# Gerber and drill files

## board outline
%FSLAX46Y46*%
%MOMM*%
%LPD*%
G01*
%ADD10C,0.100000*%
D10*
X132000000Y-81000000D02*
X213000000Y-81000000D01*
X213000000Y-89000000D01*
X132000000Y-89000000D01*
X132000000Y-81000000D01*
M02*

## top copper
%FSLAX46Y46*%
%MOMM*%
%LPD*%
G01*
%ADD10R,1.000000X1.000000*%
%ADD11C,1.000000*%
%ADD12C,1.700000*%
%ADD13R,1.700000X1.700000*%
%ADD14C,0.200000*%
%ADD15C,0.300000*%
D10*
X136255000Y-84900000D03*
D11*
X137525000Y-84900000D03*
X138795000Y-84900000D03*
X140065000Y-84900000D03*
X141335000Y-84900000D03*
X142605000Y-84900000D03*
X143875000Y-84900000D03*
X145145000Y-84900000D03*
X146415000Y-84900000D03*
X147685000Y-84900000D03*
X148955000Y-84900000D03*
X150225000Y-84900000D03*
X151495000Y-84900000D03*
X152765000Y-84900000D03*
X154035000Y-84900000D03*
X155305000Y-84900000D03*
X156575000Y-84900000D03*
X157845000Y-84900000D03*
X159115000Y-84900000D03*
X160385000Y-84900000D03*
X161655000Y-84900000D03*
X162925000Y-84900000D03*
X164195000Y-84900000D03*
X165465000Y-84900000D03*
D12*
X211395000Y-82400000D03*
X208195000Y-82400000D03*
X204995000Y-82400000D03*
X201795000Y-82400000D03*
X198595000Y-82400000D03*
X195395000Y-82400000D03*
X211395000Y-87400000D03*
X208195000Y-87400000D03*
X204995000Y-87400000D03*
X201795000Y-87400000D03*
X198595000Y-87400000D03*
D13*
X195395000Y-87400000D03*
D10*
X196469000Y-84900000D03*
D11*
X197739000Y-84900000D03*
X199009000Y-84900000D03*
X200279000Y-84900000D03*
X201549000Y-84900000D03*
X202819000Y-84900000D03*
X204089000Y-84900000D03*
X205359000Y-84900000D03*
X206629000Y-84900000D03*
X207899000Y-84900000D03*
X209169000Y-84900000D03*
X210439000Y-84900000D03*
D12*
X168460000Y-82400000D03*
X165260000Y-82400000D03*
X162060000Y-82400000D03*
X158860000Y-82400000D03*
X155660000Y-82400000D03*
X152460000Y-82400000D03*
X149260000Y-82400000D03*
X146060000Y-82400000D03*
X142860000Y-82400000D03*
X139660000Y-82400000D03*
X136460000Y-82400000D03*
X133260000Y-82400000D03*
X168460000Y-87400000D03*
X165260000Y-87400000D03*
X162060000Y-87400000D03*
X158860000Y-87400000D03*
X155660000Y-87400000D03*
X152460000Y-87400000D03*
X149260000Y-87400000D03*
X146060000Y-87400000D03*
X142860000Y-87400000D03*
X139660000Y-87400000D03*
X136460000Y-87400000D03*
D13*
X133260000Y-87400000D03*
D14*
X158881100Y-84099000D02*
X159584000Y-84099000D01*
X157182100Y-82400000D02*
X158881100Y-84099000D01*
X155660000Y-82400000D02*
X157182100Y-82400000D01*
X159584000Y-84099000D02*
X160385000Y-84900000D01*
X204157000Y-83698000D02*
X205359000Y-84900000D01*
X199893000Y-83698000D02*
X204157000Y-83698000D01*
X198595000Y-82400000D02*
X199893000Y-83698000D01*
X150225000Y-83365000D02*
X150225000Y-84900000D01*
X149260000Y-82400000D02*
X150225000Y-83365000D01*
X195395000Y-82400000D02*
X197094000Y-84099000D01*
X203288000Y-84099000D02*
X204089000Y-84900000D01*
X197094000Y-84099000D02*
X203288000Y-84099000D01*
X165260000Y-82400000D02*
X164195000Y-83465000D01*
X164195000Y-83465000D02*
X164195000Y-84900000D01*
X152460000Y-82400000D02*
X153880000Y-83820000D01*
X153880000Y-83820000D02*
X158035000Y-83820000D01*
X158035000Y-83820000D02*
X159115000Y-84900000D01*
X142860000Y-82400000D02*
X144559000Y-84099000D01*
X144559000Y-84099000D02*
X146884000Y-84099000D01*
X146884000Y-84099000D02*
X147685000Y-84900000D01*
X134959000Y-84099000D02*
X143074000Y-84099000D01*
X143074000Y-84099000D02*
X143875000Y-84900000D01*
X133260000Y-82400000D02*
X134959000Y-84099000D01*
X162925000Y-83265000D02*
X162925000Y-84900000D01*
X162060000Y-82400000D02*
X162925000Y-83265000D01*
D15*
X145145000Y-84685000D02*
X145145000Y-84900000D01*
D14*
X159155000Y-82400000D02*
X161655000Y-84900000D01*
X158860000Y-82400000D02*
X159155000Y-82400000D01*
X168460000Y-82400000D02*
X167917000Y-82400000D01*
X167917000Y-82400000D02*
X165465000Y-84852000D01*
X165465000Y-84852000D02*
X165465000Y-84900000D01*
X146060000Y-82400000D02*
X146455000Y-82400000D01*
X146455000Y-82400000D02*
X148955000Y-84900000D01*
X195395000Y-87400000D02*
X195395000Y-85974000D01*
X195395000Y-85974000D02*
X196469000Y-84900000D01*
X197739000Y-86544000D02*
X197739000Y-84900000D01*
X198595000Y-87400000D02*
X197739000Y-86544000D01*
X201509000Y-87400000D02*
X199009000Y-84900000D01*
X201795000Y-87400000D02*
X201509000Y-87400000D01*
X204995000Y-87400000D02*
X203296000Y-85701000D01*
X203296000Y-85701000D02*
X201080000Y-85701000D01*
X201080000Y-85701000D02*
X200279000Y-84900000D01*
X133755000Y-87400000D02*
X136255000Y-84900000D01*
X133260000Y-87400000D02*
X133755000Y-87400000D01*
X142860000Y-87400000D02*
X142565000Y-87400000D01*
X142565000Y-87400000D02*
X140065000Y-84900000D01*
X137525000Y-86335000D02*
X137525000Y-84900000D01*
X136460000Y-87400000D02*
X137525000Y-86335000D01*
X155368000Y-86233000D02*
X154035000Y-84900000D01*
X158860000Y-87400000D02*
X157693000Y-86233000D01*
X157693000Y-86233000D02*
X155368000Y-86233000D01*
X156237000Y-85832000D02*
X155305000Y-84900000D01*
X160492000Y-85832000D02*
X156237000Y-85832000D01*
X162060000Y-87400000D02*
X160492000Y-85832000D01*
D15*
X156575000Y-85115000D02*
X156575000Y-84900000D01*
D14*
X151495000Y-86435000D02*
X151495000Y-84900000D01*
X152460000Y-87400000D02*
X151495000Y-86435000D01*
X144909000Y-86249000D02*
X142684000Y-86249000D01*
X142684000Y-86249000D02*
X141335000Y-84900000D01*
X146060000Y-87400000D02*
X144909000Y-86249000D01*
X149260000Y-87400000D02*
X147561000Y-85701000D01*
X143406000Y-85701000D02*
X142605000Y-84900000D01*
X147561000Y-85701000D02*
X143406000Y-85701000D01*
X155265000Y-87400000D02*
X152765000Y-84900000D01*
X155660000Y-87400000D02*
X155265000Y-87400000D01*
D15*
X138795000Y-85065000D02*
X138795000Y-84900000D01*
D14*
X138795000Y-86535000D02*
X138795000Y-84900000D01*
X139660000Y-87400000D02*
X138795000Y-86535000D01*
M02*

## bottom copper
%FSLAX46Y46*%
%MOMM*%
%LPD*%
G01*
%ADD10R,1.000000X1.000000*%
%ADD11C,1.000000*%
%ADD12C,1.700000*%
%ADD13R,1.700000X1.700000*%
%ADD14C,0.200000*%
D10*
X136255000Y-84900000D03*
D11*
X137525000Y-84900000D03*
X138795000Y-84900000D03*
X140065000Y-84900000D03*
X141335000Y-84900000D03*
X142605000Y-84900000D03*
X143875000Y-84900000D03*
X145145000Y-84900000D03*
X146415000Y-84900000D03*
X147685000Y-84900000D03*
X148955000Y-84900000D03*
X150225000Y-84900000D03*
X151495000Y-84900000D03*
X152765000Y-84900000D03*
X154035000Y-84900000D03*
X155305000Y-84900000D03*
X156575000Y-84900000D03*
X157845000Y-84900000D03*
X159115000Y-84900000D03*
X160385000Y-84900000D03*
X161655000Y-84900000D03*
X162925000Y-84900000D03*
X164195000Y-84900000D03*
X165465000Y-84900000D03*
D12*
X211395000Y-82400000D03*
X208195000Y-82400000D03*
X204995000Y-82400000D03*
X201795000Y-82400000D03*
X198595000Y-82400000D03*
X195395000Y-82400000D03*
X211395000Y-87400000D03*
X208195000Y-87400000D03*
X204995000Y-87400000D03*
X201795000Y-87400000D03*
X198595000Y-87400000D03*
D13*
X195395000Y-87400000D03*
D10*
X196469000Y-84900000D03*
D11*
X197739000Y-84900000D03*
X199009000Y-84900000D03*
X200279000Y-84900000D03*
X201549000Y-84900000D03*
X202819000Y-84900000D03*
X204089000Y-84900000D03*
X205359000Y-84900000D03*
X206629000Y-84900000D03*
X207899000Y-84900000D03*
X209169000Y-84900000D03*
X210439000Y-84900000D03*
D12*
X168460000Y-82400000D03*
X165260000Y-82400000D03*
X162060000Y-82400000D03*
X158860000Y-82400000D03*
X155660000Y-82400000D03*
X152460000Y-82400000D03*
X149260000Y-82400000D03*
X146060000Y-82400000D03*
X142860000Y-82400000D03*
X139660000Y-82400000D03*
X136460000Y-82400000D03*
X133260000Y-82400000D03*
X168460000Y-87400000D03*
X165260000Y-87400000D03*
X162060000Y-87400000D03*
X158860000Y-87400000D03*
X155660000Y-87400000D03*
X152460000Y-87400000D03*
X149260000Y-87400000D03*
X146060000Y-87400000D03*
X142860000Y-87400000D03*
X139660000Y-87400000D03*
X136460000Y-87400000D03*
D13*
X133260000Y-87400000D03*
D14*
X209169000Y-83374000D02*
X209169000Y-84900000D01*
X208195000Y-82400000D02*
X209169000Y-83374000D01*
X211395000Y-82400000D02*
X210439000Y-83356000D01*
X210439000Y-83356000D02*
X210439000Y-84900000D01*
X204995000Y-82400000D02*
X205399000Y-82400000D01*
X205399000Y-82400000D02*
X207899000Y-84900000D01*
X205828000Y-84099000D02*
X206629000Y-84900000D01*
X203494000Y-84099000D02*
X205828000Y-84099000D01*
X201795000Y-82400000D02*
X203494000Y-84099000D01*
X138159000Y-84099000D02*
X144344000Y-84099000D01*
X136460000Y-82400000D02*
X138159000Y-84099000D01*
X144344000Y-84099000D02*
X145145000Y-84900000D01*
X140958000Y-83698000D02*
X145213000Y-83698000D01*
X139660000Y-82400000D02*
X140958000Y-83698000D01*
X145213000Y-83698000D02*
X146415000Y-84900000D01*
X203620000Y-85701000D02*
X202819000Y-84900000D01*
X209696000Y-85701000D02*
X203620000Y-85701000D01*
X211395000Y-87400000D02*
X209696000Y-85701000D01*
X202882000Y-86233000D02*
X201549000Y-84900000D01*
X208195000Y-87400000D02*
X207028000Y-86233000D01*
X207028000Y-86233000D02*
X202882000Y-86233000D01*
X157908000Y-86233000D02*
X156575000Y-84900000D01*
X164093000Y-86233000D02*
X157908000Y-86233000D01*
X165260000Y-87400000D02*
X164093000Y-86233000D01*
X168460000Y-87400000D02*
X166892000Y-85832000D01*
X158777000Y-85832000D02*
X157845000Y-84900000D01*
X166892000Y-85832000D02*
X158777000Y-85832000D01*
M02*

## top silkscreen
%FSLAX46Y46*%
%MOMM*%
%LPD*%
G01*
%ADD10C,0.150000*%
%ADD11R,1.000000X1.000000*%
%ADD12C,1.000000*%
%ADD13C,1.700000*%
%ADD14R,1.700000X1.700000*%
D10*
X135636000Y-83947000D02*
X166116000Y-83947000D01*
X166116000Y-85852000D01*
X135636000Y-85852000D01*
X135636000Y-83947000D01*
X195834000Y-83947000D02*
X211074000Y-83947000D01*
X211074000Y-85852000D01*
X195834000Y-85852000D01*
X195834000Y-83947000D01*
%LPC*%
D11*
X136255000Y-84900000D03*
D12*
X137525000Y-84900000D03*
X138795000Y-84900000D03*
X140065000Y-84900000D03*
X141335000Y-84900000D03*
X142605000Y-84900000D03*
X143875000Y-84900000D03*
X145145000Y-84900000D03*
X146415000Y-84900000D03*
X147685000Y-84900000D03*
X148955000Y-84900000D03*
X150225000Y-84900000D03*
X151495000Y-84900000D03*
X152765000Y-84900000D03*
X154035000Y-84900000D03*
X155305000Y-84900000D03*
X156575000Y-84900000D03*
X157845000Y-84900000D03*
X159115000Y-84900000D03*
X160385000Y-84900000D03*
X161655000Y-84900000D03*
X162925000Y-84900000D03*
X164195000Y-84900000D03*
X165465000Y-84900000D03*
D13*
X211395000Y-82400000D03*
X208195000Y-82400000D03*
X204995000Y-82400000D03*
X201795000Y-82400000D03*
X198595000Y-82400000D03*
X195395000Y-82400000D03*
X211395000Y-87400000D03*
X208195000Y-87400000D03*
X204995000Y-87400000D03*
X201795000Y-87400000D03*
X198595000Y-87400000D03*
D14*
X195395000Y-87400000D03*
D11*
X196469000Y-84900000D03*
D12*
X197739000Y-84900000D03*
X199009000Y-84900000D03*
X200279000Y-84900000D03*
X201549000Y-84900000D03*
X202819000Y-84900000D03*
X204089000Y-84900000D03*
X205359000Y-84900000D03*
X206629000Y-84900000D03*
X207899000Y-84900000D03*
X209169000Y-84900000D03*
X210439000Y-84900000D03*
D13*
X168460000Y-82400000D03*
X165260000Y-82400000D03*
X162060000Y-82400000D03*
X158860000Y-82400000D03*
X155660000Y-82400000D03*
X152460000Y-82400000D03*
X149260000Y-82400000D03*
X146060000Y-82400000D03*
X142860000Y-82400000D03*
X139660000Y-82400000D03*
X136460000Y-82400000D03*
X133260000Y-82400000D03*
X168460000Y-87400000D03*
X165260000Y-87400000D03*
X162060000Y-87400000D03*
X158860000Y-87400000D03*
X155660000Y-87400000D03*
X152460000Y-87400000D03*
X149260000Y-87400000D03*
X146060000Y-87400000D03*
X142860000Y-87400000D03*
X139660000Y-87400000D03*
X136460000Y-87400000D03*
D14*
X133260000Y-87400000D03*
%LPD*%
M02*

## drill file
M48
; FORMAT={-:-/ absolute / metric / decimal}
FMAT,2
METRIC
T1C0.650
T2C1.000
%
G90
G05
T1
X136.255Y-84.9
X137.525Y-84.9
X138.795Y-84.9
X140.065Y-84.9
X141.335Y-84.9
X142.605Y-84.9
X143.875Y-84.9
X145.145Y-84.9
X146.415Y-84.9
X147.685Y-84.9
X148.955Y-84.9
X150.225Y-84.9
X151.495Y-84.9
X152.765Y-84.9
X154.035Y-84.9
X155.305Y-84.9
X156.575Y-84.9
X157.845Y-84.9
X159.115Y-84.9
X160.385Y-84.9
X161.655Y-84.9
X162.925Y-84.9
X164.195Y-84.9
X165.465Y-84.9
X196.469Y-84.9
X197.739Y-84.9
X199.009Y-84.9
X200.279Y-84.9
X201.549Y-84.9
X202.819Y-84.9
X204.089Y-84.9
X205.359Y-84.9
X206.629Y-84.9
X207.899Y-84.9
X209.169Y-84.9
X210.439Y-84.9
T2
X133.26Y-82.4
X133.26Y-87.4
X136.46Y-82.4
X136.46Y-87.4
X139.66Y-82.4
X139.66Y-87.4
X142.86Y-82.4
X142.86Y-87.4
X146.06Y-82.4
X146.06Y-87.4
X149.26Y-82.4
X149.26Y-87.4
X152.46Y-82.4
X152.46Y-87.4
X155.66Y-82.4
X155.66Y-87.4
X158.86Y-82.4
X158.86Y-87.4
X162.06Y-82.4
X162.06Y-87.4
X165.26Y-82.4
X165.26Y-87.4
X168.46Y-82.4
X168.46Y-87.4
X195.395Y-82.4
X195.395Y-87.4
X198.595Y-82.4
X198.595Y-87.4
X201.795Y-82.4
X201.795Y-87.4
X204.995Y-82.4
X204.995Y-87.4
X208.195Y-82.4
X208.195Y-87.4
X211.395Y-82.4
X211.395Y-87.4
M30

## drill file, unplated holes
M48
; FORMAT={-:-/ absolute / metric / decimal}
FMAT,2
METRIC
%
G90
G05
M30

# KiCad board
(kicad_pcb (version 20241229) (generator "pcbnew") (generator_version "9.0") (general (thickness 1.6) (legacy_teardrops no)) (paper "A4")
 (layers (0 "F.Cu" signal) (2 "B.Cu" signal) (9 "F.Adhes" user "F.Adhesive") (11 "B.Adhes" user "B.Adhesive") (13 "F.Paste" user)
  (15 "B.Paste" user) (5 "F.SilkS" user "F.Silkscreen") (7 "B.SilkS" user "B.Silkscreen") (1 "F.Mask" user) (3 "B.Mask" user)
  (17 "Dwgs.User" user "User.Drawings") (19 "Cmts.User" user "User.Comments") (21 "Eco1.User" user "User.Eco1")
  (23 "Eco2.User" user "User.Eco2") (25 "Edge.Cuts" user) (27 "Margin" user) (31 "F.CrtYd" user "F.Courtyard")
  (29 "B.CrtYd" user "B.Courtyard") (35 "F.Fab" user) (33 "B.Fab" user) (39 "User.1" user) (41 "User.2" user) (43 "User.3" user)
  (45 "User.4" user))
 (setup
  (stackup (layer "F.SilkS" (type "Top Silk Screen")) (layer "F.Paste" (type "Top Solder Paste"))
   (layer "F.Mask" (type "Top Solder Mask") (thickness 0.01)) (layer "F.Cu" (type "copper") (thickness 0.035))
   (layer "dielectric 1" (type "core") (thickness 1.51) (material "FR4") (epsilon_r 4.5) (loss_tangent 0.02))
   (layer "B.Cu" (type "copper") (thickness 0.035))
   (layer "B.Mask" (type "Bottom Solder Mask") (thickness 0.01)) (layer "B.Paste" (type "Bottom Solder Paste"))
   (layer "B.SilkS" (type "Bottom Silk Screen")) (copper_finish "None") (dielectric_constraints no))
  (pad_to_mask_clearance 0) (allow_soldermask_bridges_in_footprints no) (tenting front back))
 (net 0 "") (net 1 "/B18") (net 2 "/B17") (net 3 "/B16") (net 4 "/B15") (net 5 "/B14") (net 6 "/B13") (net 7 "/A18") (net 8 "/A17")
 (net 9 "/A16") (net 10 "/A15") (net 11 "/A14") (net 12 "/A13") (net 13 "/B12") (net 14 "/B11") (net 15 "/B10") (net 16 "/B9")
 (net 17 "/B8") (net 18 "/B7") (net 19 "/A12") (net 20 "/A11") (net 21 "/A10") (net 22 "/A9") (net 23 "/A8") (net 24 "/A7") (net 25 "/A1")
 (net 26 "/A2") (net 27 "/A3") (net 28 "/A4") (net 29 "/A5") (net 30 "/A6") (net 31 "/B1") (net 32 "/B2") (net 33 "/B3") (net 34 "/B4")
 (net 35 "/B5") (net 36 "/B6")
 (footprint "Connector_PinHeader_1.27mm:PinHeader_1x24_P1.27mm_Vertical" (layer "F.Cu") (at 136.255 84.9 90)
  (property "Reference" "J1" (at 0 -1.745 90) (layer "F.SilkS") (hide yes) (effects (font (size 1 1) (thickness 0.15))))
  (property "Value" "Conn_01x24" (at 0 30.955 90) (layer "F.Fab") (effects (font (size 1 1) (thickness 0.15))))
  (pad "1" thru_hole rect (at 0 0 90) (size 1 1) (drill 0.65) (layers "*.Cu" "*.Mask") (remove_unused_layers no) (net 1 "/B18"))
  (pad "2" thru_hole circle (at 0 1.27 90) (size 1 1) (drill 0.65) (layers "*.Cu" "*.Mask") (remove_unused_layers no) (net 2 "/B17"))
  (pad "3" thru_hole circle (at 0 2.54 90) (size 1 1) (drill 0.65) (layers "*.Cu" "*.Mask") (remove_unused_layers no) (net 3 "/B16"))
  (pad "4" thru_hole circle (at 0 3.81 90) (size 1 1) (drill 0.65) (layers "*.Cu" "*.Mask") (remove_unused_layers no) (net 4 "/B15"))
  (pad "5" thru_hole circle (at 0 5.08 90) (size 1 1) (drill 0.65) (layers "*.Cu" "*.Mask") (remove_unused_layers no) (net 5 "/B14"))
  (pad "6" thru_hole circle (at 0 6.35 90) (size 1 1) (drill 0.65) (layers "*.Cu" "*.Mask") (remove_unused_layers no) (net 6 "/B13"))
  (pad "7" thru_hole circle (at 0 7.62 90) (size 1 1) (drill 0.65) (layers "*.Cu" "*.Mask") (remove_unused_layers no) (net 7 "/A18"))
  (pad "8" thru_hole circle (at 0 8.89 90) (size 1 1) (drill 0.65) (layers "*.Cu" "*.Mask") (remove_unused_layers no) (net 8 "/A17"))
  (pad "9" thru_hole circle (at 0 10.16 90) (size 1 1) (drill 0.65) (layers "*.Cu" "*.Mask") (remove_unused_layers no) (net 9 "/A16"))
  (pad "10" thru_hole circle (at 0 11.43 90) (size 1 1) (drill 0.65) (layers "*.Cu" "*.Mask") (remove_unused_layers no) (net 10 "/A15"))
  (pad "11" thru_hole circle (at 0 12.7 90) (size 1 1) (drill 0.65) (layers "*.Cu" "*.Mask") (remove_unused_layers no) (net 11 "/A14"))
  (pad "12" thru_hole circle (at 0 13.97 90) (size 1 1) (drill 0.65) (layers "*.Cu" "*.Mask") (remove_unused_layers no) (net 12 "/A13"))
  (pad "13" thru_hole circle (at 0 15.24 90) (size 1 1) (drill 0.65) (layers "*.Cu" "*.Mask") (remove_unused_layers no) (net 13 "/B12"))
  (pad "14" thru_hole circle (at 0 16.51 90) (size 1 1) (drill 0.65) (layers "*.Cu" "*.Mask") (remove_unused_layers no) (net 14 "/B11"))
  (pad "15" thru_hole circle (at 0 17.78 90) (size 1 1) (drill 0.65) (layers "*.Cu" "*.Mask") (remove_unused_layers no) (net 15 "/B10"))
  (pad "16" thru_hole circle (at 0 19.05 90) (size 1 1) (drill 0.65) (layers "*.Cu" "*.Mask") (remove_unused_layers no) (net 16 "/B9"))
  (pad "17" thru_hole circle (at 0 20.32 90) (size 1 1) (drill 0.65) (layers "*.Cu" "*.Mask") (remove_unused_layers no) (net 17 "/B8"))
  (pad "18" thru_hole circle (at 0 21.59 90) (size 1 1) (drill 0.65) (layers "*.Cu" "*.Mask") (remove_unused_layers no) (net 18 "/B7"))
  (pad "19" thru_hole circle (at 0 22.86 90) (size 1 1) (drill 0.65) (layers "*.Cu" "*.Mask") (remove_unused_layers no) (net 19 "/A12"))
  (pad "20" thru_hole circle (at 0 24.13 90) (size 1 1) (drill 0.65) (layers "*.Cu" "*.Mask") (remove_unused_layers no) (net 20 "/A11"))
  (pad "21" thru_hole circle (at 0 25.4 90) (size 1 1) (drill 0.65) (layers "*.Cu" "*.Mask") (remove_unused_layers no) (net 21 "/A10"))
  (pad "22" thru_hole circle (at 0 26.67 90) (size 1 1) (drill 0.65) (layers "*.Cu" "*.Mask") (remove_unused_layers no) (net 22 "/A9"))
  (pad "23" thru_hole circle (at 0 27.94 90) (size 1 1) (drill 0.65) (layers "*.Cu" "*.Mask") (remove_unused_layers no) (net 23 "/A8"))
  (pad "24" thru_hole circle (at 0 29.21 90) (size 1 1) (drill 0.65) (layers "*.Cu" "*.Mask") (remove_unused_layers no) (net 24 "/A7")))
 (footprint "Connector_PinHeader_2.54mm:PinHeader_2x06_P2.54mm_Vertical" (layer "F.Cu") (at 195.395 87.4 90)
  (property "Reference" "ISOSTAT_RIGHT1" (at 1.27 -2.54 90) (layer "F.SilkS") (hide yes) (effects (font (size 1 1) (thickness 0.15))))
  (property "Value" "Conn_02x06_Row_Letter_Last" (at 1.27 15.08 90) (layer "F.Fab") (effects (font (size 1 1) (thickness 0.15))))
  (pad "A1" thru_hole circle (at 5 16 90) (size 1.7 1.7) (drill 1) (layers "*.Cu" "*.Mask") (remove_unused_layers no) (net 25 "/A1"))
  (pad "A2" thru_hole circle (at 5 12.8 90) (size 1.7 1.7) (drill 1) (layers "*.Cu" "*.Mask") (remove_unused_layers no) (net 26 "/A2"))
  (pad "A3" thru_hole circle (at 5 9.6 90) (size 1.7 1.7) (drill 1) (layers "*.Cu" "*.Mask") (remove_unused_layers no) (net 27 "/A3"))
  (pad "A4" thru_hole circle (at 5 6.4 90) (size 1.7 1.7) (drill 1) (layers "*.Cu" "*.Mask") (remove_unused_layers no) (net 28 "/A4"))
  (pad "A5" thru_hole circle (at 5 3.2 90) (size 1.7 1.7) (drill 1) (layers "*.Cu" "*.Mask") (remove_unused_layers no) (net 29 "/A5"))
  (pad "A6" thru_hole circle (at 5 0 90) (size 1.7 1.7) (drill 1) (layers "*.Cu" "*.Mask") (remove_unused_layers no) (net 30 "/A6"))
  (pad "B1" thru_hole circle (at 0 16 90) (size 1.7 1.7) (drill 1) (layers "*.Cu" "*.Mask") (remove_unused_layers no) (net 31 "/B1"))
  (pad "B2" thru_hole circle (at 0 12.8 90) (size 1.7 1.7) (drill 1) (layers "*.Cu" "*.Mask") (remove_unused_layers no) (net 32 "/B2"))
  (pad "B3" thru_hole circle (at 0 9.6 90) (size 1.7 1.7) (drill 1) (layers "*.Cu" "*.Mask") (remove_unused_layers no) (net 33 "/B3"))
  (pad "B4" thru_hole circle (at 0 6.4 90) (size 1.7 1.7) (drill 1) (layers "*.Cu" "*.Mask") (remove_unused_layers no) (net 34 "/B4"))
  (pad "B5" thru_hole circle (at 0 3.2 90) (size 1.7 1.7) (drill 1) (layers "*.Cu" "*.Mask") (remove_unused_layers no) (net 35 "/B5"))
  (pad "B6" thru_hole rect (at 0 0 90) (size 1.7 1.7) (drill 1) (layers "*.Cu" "*.Mask") (remove_unused_layers no) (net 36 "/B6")))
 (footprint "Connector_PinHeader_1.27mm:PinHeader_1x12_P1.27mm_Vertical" (layer "F.Cu") (at 196.469 84.9 90)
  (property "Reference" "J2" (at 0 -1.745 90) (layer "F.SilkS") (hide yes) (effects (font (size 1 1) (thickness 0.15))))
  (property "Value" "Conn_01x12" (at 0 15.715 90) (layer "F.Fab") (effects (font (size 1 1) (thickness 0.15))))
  (pad "1" thru_hole rect (at 0 0 90) (size 1 1) (drill 0.65) (layers "*.Cu" "*.Mask") (remove_unused_layers no) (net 36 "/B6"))
  (pad "2" thru_hole circle (at 0 1.27 90) (size 1 1) (drill 0.65) (layers "*.Cu" "*.Mask") (remove_unused_layers no) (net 35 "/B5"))
  (pad "3" thru_hole circle (at 0 2.54 90) (size 1 1) (drill 0.65) (layers "*.Cu" "*.Mask") (remove_unused_layers no) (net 34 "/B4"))
  (pad "4" thru_hole circle (at 0 3.81 90) (size 1 1) (drill 0.65) (layers "*.Cu" "*.Mask") (remove_unused_layers no) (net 33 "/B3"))
  (pad "5" thru_hole circle (at 0 5.08 90) (size 1 1) (drill 0.65) (layers "*.Cu" "*.Mask") (remove_unused_layers no) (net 32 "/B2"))
  (pad "6" thru_hole circle (at 0 6.35 90) (size 1 1) (drill 0.65) (layers "*.Cu" "*.Mask") (remove_unused_layers no) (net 31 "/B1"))
  (pad "7" thru_hole circle (at 0 7.62 90) (size 1 1) (drill 0.65) (layers "*.Cu" "*.Mask") (remove_unused_layers no) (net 30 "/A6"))
  (pad "8" thru_hole circle (at 0 8.89 90) (size 1 1) (drill 0.65) (layers "*.Cu" "*.Mask") (remove_unused_layers no) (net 29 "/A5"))
  (pad "9" thru_hole circle (at 0 10.16 90) (size 1 1) (drill 0.65) (layers "*.Cu" "*.Mask") (remove_unused_layers no) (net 28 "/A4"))
  (pad "10" thru_hole circle (at 0 11.43 90) (size 1 1) (drill 0.65) (layers "*.Cu" "*.Mask") (remove_unused_layers no) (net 27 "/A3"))
  (pad "11" thru_hole circle (at 0 12.7 90) (size 1 1) (drill 0.65) (layers "*.Cu" "*.Mask") (remove_unused_layers no) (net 26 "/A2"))
  (pad "12" thru_hole circle (at 0 13.97 90) (size 1 1) (drill 0.65) (layers "*.Cu" "*.Mask") (remove_unused_layers no) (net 25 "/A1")))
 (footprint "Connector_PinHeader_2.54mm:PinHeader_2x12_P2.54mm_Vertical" (layer "F.Cu") (at 133.26 87.4 90)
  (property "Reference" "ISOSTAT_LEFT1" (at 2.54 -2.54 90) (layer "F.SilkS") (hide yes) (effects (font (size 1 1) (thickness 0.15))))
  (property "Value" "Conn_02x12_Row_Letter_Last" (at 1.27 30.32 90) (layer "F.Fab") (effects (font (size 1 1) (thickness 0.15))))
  (pad "A7" thru_hole circle (at 5 35.2 90) (size 1.7 1.7) (drill 1) (layers "*.Cu" "*.Mask") (remove_unused_layers no) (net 24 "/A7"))
  (pad "A8" thru_hole circle (at 5 32 90) (size 1.7 1.7) (drill 1) (layers "*.Cu" "*.Mask") (remove_unused_layers no) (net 23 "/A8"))
  (pad "A9" thru_hole circle (at 5 28.8 90) (size 1.7 1.7) (drill 1) (layers "*.Cu" "*.Mask") (remove_unused_layers no) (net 22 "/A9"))
  (pad "A10" thru_hole circle (at 5 25.6 90) (size 1.7 1.7) (drill 1) (layers "*.Cu" "*.Mask") (remove_unused_layers no) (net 21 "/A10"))
  (pad "A11" thru_hole circle (at 5 22.4 90) (size 1.7 1.7) (drill 1) (layers "*.Cu" "*.Mask") (remove_unused_layers no) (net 20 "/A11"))
  (pad "A12" thru_hole circle (at 5 19.2 90) (size 1.7 1.7) (drill 1) (layers "*.Cu" "*.Mask") (remove_unused_layers no) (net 19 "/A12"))
  (pad "A13" thru_hole circle (at 5 16 90) (size 1.7 1.7) (drill 1) (layers "*.Cu" "*.Mask") (remove_unused_layers no) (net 12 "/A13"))
  (pad "A14" thru_hole circle (at 5 12.8 90) (size 1.7 1.7) (drill 1) (layers "*.Cu" "*.Mask") (remove_unused_layers no) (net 11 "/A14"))
  (pad "A15" thru_hole circle (at 5 9.6 90) (size 1.7 1.7) (drill 1) (layers "*.Cu" "*.Mask") (remove_unused_layers no) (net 10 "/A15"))
  (pad "A16" thru_hole circle (at 5 6.4 90) (size 1.7 1.7) (drill 1) (layers "*.Cu" "*.Mask") (remove_unused_layers no) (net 9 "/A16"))
  (pad "A17" thru_hole circle (at 5 3.2 90) (size 1.7 1.7) (drill 1) (layers "*.Cu" "*.Mask") (remove_unused_layers no) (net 8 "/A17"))
  (pad "A18" thru_hole circle (at 5 0 90) (size 1.7 1.7) (drill 1) (layers "*.Cu" "*.Mask") (remove_unused_layers no) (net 7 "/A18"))
  (pad "B7" thru_hole circle (at 0 35.2 90) (size 1.7 1.7) (drill 1) (layers "*.Cu" "*.Mask") (remove_unused_layers no) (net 18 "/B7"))
  (pad "B8" thru_hole circle (at 0 32 90) (size 1.7 1.7) (drill 1) (layers "*.Cu" "*.Mask") (remove_unused_layers no) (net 17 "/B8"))
  (pad "B9" thru_hole circle (at 0 28.8 90) (size 1.7 1.7) (drill 1) (layers "*.Cu" "*.Mask") (remove_unused_layers no) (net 16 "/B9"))
  (pad "B10" thru_hole circle (at 0 25.6 90) (size 1.7 1.7) (drill 1) (layers "*.Cu" "*.Mask") (remove_unused_layers no) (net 15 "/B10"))
  (pad "B11" thru_hole circle (at 0 22.4 90) (size 1.7 1.7) (drill 1) (layers "*.Cu" "*.Mask") (remove_unused_layers no) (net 14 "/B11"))
  (pad "B12" thru_hole circle (at 0 19.2 90) (size 1.7 1.7) (drill 1) (layers "*.Cu" "*.Mask") (remove_unused_layers no) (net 13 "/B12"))
  (pad "B13" thru_hole circle (at 0 16 90) (size 1.7 1.7) (drill 1) (layers "*.Cu" "*.Mask") (remove_unused_layers no) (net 6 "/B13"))
  (pad "B14" thru_hole circle (at 0 12.8 90) (size 1.7 1.7) (drill 1) (layers "*.Cu" "*.Mask") (remove_unused_layers no) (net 5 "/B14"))
  (pad "B15" thru_hole circle (at 0 9.6 90) (size 1.7 1.7) (drill 1) (layers "*.Cu" "*.Mask") (remove_unused_layers no) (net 4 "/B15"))
  (pad "B16" thru_hole circle (at 0 6.4 180) (size 1.7 1.7) (drill 1) (layers "*.Cu" "*.Mask") (remove_unused_layers no) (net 3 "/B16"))
  (pad "B17" thru_hole circle (at 0 3.2 90) (size 1.7 1.7) (drill 1) (layers "*.Cu" "*.Mask") (remove_unused_layers no) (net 2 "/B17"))
  (pad "B18" thru_hole rect (at 0 0 90) (size 1.7 1.7) (drill 1) (layers "*.Cu" "*.Mask") (remove_unused_layers no) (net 1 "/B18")))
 (gr_rect (start 135.636 83.947) (end 166.116 85.852) (stroke (width 0.15) (type default)) (fill no) (layer "F.SilkS"))
 (gr_rect (start 195.834 83.947) (end 211.074 85.852) (stroke (width 0.15) (type default)) (fill no) (layer "F.SilkS"))
 (gr_rect (start 132 81) (end 213 89) (stroke (width 0.1) (type default)) (fill no) (layer "Edge.Cuts"))
 (segment (start 158.8811 84.099) (end 159.584 84.099) (width 0.2) (layer "F.Cu") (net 20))
 (segment (start 157.1821 82.4) (end 158.8811 84.099) (width 0.2) (layer "F.Cu") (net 20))
 (segment (start 155.66 82.4) (end 157.1821 82.4) (width 0.2) (layer "F.Cu") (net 20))
 (segment (start 159.584 84.099) (end 160.385 84.9) (width 0.2) (layer "F.Cu") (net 20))
 (segment (start 204.157 83.698) (end 205.359 84.9) (width 0.2) (layer "F.Cu") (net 29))
 (segment (start 199.893 83.698) (end 204.157 83.698) (width 0.2) (layer "F.Cu") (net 29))
 (segment (start 198.595 82.4) (end 199.893 83.698) (width 0.2) (layer "F.Cu") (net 29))
 (segment (start 209.169 83.374) (end 209.169 84.9) (width 0.2) (layer "B.Cu") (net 26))
 (segment (start 208.195 82.4) (end 209.169 83.374) (width 0.2) (layer "B.Cu") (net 26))
 (segment (start 150.225 83.365) (end 150.225 84.9) (width 0.2) (layer "F.Cu") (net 12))
 (segment (start 149.26 82.4) (end 150.225 83.365) (width 0.2) (layer "F.Cu") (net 12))
 (segment (start 195.395 82.4) (end 197.094 84.099) (width 0.2) (layer "F.Cu") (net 30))
 (segment (start 203.288 84.099) (end 204.089 84.9) (width 0.2) (layer "F.Cu") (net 30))
 (segment (start 197.094 84.099) (end 203.288 84.099) (width 0.2) (layer "F.Cu") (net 30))
 (segment (start 165.26 82.4) (end 164.195 83.465) (width 0.2) (layer "F.Cu") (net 23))
 (segment (start 164.195 83.465) (end 164.195 84.9) (width 0.2) (layer "F.Cu") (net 23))
 (segment (start 211.395 82.4) (end 210.439 83.356) (width 0.2) (layer "B.Cu") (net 25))
 (segment (start 210.439 83.356) (end 210.439 84.9) (width 0.2) (layer "B.Cu") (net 25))
 (segment (start 152.46 82.4) (end 153.88 83.82) (width 0.2) (layer "F.Cu") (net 19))
 (segment (start 153.88 83.82) (end 158.035 83.82) (width 0.2) (layer "F.Cu") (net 19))
 (segment (start 158.035 83.82) (end 159.115 84.9) (width 0.2) (layer "F.Cu") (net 19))
 (segment (start 142.86 82.4) (end 144.559 84.099) (width 0.2) (layer "F.Cu") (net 10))
 (segment (start 144.559 84.099) (end 146.884 84.099) (width 0.2) (layer "F.Cu") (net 10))
 (segment (start 146.884 84.099) (end 147.685 84.9) (width 0.2) (layer "F.Cu") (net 10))
 (segment (start 134.959 84.099) (end 143.074 84.099) (width 0.2) (layer "F.Cu") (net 7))
 (segment (start 143.074 84.099) (end 143.875 84.9) (width 0.2) (layer "F.Cu") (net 7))
 (segment (start 133.26 82.4) (end 134.959 84.099) (width 0.2) (layer "F.Cu") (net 7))
 (segment (start 204.995 82.4) (end 205.399 82.4) (width 0.2) (layer "B.Cu") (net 27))
 (segment (start 205.399 82.4) (end 207.899 84.9) (width 0.2) (layer "B.Cu") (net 27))
 (segment (start 205.828 84.099) (end 206.629 84.9) (width 0.2) (layer "B.Cu") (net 28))
 (segment (start 203.494 84.099) (end 205.828 84.099) (width 0.2) (layer "B.Cu") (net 28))
 (segment (start 201.795 82.4) (end 203.494 84.099) (width 0.2) (layer "B.Cu") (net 28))
 (segment (start 162.925 83.265) (end 162.925 84.9) (width 0.2) (layer "F.Cu") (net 22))
 (segment (start 162.06 82.4) (end 162.925 83.265) (width 0.2) (layer "F.Cu") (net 22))
 (segment (start 145.145 84.685) (end 145.145 84.9) (width 0.3) (layer "F.Cu") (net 8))
 (segment (start 138.159 84.099) (end 144.344 84.099) (width 0.2) (layer "B.Cu") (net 8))
 (segment (start 136.46 82.4) (end 138.159 84.099) (width 0.2) (layer "B.Cu") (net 8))
 (segment (start 144.344 84.099) (end 145.145 84.9) (width 0.2) (layer "B.Cu") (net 8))
 (segment (start 159.155 82.4) (end 161.655 84.9) (width 0.2) (layer "F.Cu") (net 21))
 (segment (start 158.86 82.4) (end 159.155 82.4) (width 0.2) (layer "F.Cu") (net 21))
 (segment (start 168.46 82.4) (end 167.917 82.4) (width 0.2) (layer "F.Cu") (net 24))
 (segment (start 167.917 82.4) (end 165.465 84.852) (width 0.2) (layer "F.Cu") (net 24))
 (segment (start 165.465 84.852) (end 165.465 84.9) (width 0.2) (layer "F.Cu") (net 24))
 (segment (start 140.958 83.698) (end 145.213 83.698) (width 0.2) (layer "B.Cu") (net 9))
 (segment (start 139.66 82.4) (end 140.958 83.698) (width 0.2) (layer "B.Cu") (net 9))
 (segment (start 145.213 83.698) (end 146.415 84.9) (width 0.2) (layer "B.Cu") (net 9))
 (segment (start 146.06 82.4) (end 146.455 82.4) (width 0.2) (layer "F.Cu") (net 11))
 (segment (start 146.455 82.4) (end 148.955 84.9) (width 0.2) (layer "F.Cu") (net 11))
 (segment (start 203.62 85.701) (end 202.819 84.9) (width 0.2) (layer "B.Cu") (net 31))
 (segment (start 209.696 85.701) (end 203.62 85.701) (width 0.2) (layer "B.Cu") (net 31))
 (segment (start 211.395 87.4) (end 209.696 85.701) (width 0.2) (layer "B.Cu") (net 31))
 (segment (start 195.395 87.4) (end 195.395 85.974) (width 0.2) (layer "F.Cu") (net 36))
 (segment (start 195.395 85.974) (end 196.469 84.9) (width 0.2) (layer "F.Cu") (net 36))
 (segment (start 202.882 86.233) (end 201.549 84.9) (width 0.2) (layer "B.Cu") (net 32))
 (segment (start 208.195 87.4) (end 207.028 86.233) (width 0.2) (layer "B.Cu") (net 32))
 (segment (start 207.028 86.233) (end 202.882 86.233) (width 0.2) (layer "B.Cu") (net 32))
 (segment (start 197.739 86.544) (end 197.739 84.9) (width 0.2) (layer "F.Cu") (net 35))
 (segment (start 198.595 87.4) (end 197.739 86.544) (width 0.2) (layer "F.Cu") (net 35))
 (segment (start 201.509 87.4) (end 199.009 84.9) (width 0.2) (layer "F.Cu") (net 34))
 (segment (start 201.795 87.4) (end 201.509 87.4) (width 0.2) (layer "F.Cu") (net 34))
 (segment (start 204.995 87.4) (end 203.296 85.701) (width 0.2) (layer "F.Cu") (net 33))
 (segment (start 203.296 85.701) (end 201.08 85.701) (width 0.2) (layer "F.Cu") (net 33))
 (segment (start 201.08 85.701) (end 200.279 84.9) (width 0.2) (layer "F.Cu") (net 33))
 (segment (start 133.755 87.4) (end 136.255 84.9) (width 0.2) (layer "F.Cu") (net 1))
 (segment (start 133.26 87.4) (end 133.755 87.4) (width 0.2) (layer "F.Cu") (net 1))
 (segment (start 142.86 87.4) (end 142.565 87.4) (width 0.2) (layer "F.Cu") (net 4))
 (segment (start 142.565 87.4) (end 140.065 84.9) (width 0.2) (layer "F.Cu") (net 4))
 (segment (start 137.525 86.335) (end 137.525 84.9) (width 0.2) (layer "F.Cu") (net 2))
 (segment (start 136.46 87.4) (end 137.525 86.335) (width 0.2) (layer "F.Cu") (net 2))
 (segment (start 155.368 86.233) (end 154.035 84.9) (width 0.2) (layer "F.Cu") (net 15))
 (segment (start 158.86 87.4) (end 157.693 86.233) (width 0.2) (layer "F.Cu") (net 15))
 (segment (start 157.693 86.233) (end 155.368 86.233) (width 0.2) (layer "F.Cu") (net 15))
 (segment (start 156.237 85.832) (end 155.305 84.9) (width 0.2) (layer "F.Cu") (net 16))
 (segment (start 160.492 85.832) (end 156.237 85.832) (width 0.2) (layer "F.Cu") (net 16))
 (segment (start 162.06 87.4) (end 160.492 85.832) (width 0.2) (layer "F.Cu") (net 16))
 (segment (start 156.575 85.115) (end 156.575 84.9) (width 0.3) (layer "F.Cu") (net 17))
 (segment (start 157.908 86.233) (end 156.575 84.9) (width 0.2) (layer "B.Cu") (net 17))
 (segment (start 164.093 86.233) (end 157.908 86.233) (width 0.2) (layer "B.Cu") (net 17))
 (segment (start 165.26 87.4) (end 164.093 86.233) (width 0.2) (layer "B.Cu") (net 17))
 (segment (start 151.495 86.435) (end 151.495 84.9) (width 0.2) (layer "F.Cu") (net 13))
 (segment (start 152.46 87.4) (end 151.495 86.435) (width 0.2) (layer "F.Cu") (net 13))
 (segment (start 144.909 86.249) (end 142.684 86.249) (width 0.2) (layer "F.Cu") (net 5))
 (segment (start 142.684 86.249) (end 141.335 84.9) (width 0.2) (layer "F.Cu") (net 5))
 (segment (start 146.06 87.4) (end 144.909 86.249) (width 0.2) (layer "F.Cu") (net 5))
 (segment (start 168.46 87.4) (end 166.892 85.832) (width 0.2) (layer "B.Cu") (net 18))
 (segment (start 158.777 85.832) (end 157.845 84.9) (width 0.2) (layer "B.Cu") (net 18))
 (segment (start 166.892 85.832) (end 158.777 85.832) (width 0.2) (layer "B.Cu") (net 18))
 (segment (start 149.26 87.4) (end 147.561 85.701) (width 0.2) (layer "F.Cu") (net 6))
 (segment (start 143.406 85.701) (end 142.605 84.9) (width 0.2) (layer "F.Cu") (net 6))
 (segment (start 147.561 85.701) (end 143.406 85.701) (width 0.2) (layer "F.Cu") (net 6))
 (segment (start 155.265 87.4) (end 152.765 84.9) (width 0.2) (layer "F.Cu") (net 14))
 (segment (start 155.66 87.4) (end 155.265 87.4) (width 0.2) (layer "F.Cu") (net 14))
 (segment (start 138.795 85.065) (end 138.795 84.9) (width 0.3) (layer "F.Cu") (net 3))
 (segment (start 138.795 86.535) (end 138.795 84.9) (width 0.2) (layer "F.Cu") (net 3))
 (segment (start 139.66 87.4) (end 138.795 86.535) (width 0.2) (layer "F.Cu") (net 3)))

